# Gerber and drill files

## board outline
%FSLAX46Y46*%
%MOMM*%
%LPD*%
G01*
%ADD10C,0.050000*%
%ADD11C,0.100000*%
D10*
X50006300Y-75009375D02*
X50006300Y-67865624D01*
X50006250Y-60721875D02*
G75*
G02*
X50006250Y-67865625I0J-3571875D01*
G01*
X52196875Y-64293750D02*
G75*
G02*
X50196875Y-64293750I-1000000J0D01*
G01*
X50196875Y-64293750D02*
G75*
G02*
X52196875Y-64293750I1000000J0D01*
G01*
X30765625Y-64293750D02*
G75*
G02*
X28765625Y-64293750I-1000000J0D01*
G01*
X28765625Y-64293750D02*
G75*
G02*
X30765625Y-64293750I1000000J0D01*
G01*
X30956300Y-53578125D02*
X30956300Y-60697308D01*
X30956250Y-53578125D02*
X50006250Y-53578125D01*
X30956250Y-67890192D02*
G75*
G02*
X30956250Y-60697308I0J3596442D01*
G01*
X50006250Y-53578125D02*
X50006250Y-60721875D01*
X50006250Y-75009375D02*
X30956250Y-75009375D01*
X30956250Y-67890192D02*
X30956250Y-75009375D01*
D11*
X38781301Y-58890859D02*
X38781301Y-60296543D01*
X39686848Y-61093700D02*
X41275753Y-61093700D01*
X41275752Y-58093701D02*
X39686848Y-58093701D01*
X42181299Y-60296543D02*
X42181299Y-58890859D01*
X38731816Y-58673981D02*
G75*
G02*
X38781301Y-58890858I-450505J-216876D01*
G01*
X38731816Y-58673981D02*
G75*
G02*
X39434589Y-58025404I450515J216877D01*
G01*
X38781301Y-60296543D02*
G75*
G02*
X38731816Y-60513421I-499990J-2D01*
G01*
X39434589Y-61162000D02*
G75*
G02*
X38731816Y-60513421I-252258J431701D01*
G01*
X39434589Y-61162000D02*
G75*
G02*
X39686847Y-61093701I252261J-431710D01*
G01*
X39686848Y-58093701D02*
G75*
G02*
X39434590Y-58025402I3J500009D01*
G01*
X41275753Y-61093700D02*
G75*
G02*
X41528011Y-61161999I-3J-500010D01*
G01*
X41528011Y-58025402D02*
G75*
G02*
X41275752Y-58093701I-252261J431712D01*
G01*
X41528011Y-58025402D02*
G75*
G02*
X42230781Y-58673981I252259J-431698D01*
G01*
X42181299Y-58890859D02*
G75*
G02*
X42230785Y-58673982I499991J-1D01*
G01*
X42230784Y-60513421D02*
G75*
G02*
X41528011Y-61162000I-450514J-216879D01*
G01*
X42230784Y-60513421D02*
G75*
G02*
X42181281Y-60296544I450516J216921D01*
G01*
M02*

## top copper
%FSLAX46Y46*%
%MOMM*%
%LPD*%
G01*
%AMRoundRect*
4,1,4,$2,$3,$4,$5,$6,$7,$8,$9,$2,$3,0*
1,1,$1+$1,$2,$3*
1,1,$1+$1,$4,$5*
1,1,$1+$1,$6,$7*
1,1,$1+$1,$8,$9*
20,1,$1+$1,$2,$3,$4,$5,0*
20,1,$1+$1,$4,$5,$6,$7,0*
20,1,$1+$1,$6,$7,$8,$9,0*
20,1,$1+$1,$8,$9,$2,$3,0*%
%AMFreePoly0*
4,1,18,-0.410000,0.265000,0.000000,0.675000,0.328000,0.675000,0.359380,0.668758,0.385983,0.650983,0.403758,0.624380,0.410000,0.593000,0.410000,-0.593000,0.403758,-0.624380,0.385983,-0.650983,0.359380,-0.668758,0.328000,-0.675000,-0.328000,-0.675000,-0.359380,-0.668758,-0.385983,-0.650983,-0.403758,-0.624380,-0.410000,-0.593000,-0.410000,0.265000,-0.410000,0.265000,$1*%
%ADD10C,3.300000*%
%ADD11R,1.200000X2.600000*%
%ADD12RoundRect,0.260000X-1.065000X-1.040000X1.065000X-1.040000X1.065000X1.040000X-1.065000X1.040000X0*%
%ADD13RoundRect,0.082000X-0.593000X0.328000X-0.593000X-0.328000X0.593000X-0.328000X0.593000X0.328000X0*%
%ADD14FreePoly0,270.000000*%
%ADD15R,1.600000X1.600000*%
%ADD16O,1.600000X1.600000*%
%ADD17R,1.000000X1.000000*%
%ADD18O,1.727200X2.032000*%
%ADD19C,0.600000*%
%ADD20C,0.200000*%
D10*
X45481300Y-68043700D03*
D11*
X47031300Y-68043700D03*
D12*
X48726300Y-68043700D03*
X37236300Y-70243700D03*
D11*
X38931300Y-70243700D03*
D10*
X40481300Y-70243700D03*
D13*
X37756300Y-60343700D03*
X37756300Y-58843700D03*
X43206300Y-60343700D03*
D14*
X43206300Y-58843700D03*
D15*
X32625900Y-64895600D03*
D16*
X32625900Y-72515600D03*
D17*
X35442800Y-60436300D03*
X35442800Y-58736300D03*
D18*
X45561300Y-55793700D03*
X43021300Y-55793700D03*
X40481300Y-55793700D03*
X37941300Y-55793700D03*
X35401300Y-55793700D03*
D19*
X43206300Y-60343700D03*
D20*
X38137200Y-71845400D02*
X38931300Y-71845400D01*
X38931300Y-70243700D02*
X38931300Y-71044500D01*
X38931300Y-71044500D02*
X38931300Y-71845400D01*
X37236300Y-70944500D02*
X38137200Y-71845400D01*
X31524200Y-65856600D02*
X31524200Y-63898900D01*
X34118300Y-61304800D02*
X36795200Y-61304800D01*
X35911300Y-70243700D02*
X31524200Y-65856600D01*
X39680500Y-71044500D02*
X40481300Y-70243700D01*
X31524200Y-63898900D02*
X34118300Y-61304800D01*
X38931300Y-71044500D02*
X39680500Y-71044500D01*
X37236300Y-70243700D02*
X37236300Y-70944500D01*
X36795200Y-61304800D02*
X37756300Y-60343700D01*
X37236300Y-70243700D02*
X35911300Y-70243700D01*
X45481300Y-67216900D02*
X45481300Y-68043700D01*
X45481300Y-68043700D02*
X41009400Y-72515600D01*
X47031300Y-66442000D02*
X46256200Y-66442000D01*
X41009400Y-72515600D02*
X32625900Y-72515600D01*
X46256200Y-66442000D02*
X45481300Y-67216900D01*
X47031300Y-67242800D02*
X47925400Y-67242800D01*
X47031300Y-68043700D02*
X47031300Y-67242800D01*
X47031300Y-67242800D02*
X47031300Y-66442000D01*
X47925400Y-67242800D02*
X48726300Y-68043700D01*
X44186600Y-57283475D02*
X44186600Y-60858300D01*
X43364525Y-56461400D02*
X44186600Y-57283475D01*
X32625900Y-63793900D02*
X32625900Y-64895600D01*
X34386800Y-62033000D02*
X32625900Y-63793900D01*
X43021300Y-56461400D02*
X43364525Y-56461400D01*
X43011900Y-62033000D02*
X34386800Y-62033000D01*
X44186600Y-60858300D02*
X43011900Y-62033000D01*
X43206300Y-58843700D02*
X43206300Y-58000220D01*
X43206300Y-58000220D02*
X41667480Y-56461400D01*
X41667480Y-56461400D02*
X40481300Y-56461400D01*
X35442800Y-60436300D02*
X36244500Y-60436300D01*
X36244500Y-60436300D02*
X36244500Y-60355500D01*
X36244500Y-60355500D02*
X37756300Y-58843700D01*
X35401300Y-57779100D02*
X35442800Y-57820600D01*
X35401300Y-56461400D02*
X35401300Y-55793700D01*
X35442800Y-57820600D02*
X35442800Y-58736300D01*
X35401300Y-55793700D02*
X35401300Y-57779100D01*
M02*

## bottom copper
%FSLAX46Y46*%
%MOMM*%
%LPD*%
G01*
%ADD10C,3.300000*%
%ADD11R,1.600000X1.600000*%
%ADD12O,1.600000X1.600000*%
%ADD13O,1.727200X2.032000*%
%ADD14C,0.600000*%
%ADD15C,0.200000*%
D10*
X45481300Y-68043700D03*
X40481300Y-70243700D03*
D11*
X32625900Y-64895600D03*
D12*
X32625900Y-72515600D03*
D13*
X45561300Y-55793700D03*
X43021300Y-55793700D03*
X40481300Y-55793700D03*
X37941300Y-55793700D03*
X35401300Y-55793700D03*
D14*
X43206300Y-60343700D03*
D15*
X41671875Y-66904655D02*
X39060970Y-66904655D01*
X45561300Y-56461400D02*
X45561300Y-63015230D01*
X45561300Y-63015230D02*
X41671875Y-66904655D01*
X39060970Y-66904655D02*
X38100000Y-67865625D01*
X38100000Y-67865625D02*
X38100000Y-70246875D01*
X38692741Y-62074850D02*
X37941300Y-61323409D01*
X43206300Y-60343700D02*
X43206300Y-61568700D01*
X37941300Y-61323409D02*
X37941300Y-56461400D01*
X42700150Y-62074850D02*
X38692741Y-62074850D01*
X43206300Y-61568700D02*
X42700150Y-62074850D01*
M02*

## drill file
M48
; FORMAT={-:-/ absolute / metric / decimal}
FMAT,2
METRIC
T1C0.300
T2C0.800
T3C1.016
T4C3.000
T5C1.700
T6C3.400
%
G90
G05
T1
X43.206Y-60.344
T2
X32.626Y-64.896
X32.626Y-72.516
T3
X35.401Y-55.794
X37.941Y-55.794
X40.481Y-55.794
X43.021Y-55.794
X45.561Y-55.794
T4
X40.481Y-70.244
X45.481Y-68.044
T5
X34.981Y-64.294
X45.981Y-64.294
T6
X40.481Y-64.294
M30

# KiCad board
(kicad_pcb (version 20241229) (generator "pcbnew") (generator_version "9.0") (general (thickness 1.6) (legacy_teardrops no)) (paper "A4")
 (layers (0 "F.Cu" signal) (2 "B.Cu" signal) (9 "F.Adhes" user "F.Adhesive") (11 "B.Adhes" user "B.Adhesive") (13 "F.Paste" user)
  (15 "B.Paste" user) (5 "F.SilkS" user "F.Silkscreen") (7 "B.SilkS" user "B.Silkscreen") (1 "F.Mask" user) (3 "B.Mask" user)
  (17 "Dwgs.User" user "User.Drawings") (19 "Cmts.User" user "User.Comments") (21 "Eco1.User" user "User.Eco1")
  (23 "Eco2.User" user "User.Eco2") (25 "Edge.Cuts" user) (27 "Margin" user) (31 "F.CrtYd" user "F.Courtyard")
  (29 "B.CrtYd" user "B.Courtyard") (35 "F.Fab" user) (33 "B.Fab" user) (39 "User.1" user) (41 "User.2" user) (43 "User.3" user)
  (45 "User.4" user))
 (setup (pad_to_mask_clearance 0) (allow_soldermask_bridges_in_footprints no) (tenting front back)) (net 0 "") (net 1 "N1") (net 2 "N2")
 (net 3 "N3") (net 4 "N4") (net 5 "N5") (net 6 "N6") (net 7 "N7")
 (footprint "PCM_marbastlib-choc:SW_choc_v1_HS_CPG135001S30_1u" (layer "F.Cu") (at 40.4813 64.2937)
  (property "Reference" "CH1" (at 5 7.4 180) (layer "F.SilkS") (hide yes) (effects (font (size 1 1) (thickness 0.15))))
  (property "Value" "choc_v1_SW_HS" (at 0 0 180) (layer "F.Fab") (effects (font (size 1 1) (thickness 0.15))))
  (pad "" np_thru_hole circle (at -5.5 0 180) (size 1.7 1.7) (drill 1.7) (layers "*.Cu" "*.Mask"))
  (pad "" np_thru_hole circle (at 0 0 180) (size 3.4 3.4) (drill 3.4) (layers "*.Cu" "*.Mask"))
  (pad "" np_thru_hole circle (at 5.5 0 180) (size 1.7 1.7) (drill 1.7) (layers "*.Cu" "*.Mask"))
  (pad "1" thru_hole circle (at 5 3.75) (size 3.3 3.3) (drill 3) (layers "*.Cu" "F.Mask") (remove_unused_layers no) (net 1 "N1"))
  (pad "1" smd rect (at 6.55 3.75) (size 1.2 2.6) (layers "F.Cu") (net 1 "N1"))
  (pad "1" smd roundrect (at 8.245 3.75) (size 2.65 2.6) (layers "F.Cu" "F.Mask" "F.Paste") (roundrect_rratio 0.1) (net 1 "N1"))
  (pad "2" smd roundrect (at -3.245 5.95) (size 2.65 2.6) (layers "F.Cu" "F.Mask" "F.Paste") (roundrect_rratio 0.1) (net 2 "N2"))
  (pad "2" smd rect (at -1.55 5.95 180) (size 1.2 2.6) (layers "F.Cu") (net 2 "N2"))
  (pad "2" thru_hole circle (at 0 5.95) (size 3.3 3.3) (drill 3) (layers "*.Cu" "F.Mask") (remove_unused_layers no) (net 2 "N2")))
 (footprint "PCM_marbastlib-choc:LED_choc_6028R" (layer "F.Cu") (at 40.4813 59.5937)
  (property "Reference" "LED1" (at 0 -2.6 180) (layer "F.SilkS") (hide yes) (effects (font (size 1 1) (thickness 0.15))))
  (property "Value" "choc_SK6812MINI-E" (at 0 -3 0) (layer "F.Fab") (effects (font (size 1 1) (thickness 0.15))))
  (fp_line (start -1.699999 -0.702841) (end -1.699999 0.702843) (stroke (width 0.1) (type solid)) (layer "Edge.Cuts"))
  (fp_line (start -0.794452 1.5) (end 0.794453 1.5) (stroke (width 0.1) (type solid)) (layer "Edge.Cuts"))
  (fp_line (start 0.794452 -1.499999) (end -0.794452 -1.499999) (stroke (width 0.1) (type solid)) (layer "Edge.Cuts"))
  (fp_line (start 1.699999 0.702843) (end 1.699999 -0.702841) (stroke (width 0.1) (type solid)) (layer "Edge.Cuts"))
  (fp_arc (start -1.749484 -0.919719) (mid -1.712527 -0.814067) (end -1.699999 -0.702842) (stroke (width 0.1) (type solid))
   (layer "Edge.Cuts"))
  (fp_arc (start -1.749484 -0.919719) (mid -1.63807 -1.504033) (end -1.046711 -1.568296) (stroke (width 0.1) (type solid))
   (layer "Edge.Cuts"))
  (fp_arc (start -1.699999 0.702843) (mid -1.712527 0.814069) (end -1.749484 0.919721) (stroke (width 0.1) (type solid)) (layer "Edge.Cuts"))
  (fp_arc (start -1.046711 1.5683) (mid -1.638071 1.504036) (end -1.749484 0.919721) (stroke (width 0.1) (type solid)) (layer "Edge.Cuts"))
  (fp_arc (start -1.046711 1.5683) (mid -0.925123 1.517378) (end -0.794453 1.500001) (stroke (width 0.1) (type solid)) (layer "Edge.Cuts"))
  (fp_arc (start -0.794452 -1.499999) (mid -0.925122 -1.517376) (end -1.04671 -1.568298) (stroke (width 0.1) (type solid))
   (layer "Edge.Cuts"))
  (fp_arc (start 0.794453 1.5) (mid 0.925123 1.517377) (end 1.046711 1.568299) (stroke (width 0.1) (type solid)) (layer "Edge.Cuts"))
  (fp_arc (start 1.046711 -1.568298) (mid 0.925123 -1.517376) (end 0.794452 -1.499999) (stroke (width 0.1) (type solid)) (layer "Edge.Cuts"))
  (fp_arc (start 1.046711 -1.568298) (mid 1.638072 -1.504034) (end 1.749484 -0.919718) (stroke (width 0.1) (type solid)) (layer "Edge.Cuts"))
  (fp_arc (start 1.699999 -0.702841) (mid 1.712527 -0.814067) (end 1.749484 -0.919719) (stroke (width 0.1) (type solid)) (layer "Edge.Cuts"))
  (fp_arc (start 1.749484 0.919721) (mid 1.638071 1.504035) (end 1.046711 1.568299) (stroke (width 0.1) (type solid)) (layer "Edge.Cuts"))
  (fp_arc (start 1.749484 0.919721) (mid 1.712527 0.814069) (end 1.699999 0.702844) (stroke (width 0.1) (type solid)) (layer "Edge.Cuts"))
  (pad "1" smd roundrect (at -2.725 0.75 270) (size 0.82 1.35) (layers "F.Cu" "F.Mask" "F.Paste") (roundrect_rratio 0.1) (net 2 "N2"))
  (pad "2" smd roundrect (at -2.725 -0.75 270) (size 0.82 1.35) (layers "F.Cu" "F.Mask" "F.Paste") (roundrect_rratio 0.1) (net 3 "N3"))
  (pad "3" smd roundrect (at 2.725 0.75 270) (size 0.82 1.35) (layers "F.Cu" "F.Mask" "F.Paste") (roundrect_rratio 0.1) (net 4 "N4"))
  (pad "4" smd roundrect (at 2.725 -0.75 270) (size 0.82 1.35) (layers "F.Cu" "F.Mask" "F.Paste") (roundrect_rratio 0.1) (chamfer_ratio 0.5)
   (chamfer top_left) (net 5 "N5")))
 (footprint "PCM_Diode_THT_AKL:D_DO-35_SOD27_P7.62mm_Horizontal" (layer "F.Cu") (at 32.6259 64.8956 -90)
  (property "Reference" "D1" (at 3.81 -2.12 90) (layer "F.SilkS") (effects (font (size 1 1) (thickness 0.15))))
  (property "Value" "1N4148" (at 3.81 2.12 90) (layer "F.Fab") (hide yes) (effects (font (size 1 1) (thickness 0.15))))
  (pad "1" thru_hole rect (at 0 0 270) (size 1.6 1.6) (drill 0.8) (layers "*.Cu" "*.Mask") (remove_unused_layers no) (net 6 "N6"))
  (pad "2" thru_hole oval (at 7.62 0 270) (size 1.6 1.6) (drill 0.8) (layers "*.Cu" "*.Mask") (remove_unused_layers no) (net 1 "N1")))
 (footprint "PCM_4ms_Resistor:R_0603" (layer "F.Cu") (at 35.4428 59.5863 90)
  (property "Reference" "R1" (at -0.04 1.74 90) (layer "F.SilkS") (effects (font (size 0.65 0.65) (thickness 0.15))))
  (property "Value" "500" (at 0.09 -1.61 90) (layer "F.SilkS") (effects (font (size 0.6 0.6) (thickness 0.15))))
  (pad "1" smd rect (at -0.85 0 90) (size 1 1) (layers "F.Cu" "F.Mask" "F.Paste") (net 3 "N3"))
  (pad "2" smd rect (at 0.85 0 90) (size 1 1) (layers "F.Cu" "F.Mask" "F.Paste") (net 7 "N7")))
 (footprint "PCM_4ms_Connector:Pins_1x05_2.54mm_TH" (layer "B.Cu") (at 40.4813 55.7937 90)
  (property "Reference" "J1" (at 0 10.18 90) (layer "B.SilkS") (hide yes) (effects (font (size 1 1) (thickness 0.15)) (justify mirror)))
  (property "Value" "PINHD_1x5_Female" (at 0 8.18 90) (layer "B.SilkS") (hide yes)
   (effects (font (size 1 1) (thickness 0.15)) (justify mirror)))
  (pad "1" thru_hole oval (at 0 5.08 90) (size 2.032 1.7272) (drill 1.016) (layers "*.Cu" "*.Mask") (remove_unused_layers no) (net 2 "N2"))
  (pad "2" thru_hole oval (at 0 2.54 90) (size 2.032 1.7272) (drill 1.016) (layers "*.Cu" "*.Mask") (remove_unused_layers no) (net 6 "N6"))
  (pad "3" thru_hole oval (at 0 0 90) (size 2.032 1.7272) (drill 1.016) (layers "*.Cu" "*.Mask") (remove_unused_layers no) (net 5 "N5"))
  (pad "4" thru_hole oval (at 0 -2.54 90) (size 2.032 1.7272) (drill 1.016) (layers "*.Cu" "*.Mask") (remove_unused_layers no) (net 4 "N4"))
  (pad "5" thru_hole oval (at 0 -5.08 90) (size 2.032 1.7272) (drill 1.016) (layers "*.Cu" "*.Mask") (remove_unused_layers no) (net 7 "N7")))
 (gr_line (start 50.0063 75.009375) (end 50.0063 67.865624) (stroke (width 0.05) (type default)) (layer "Edge.Cuts"))
 (gr_arc (start 50.00625 60.721875) (mid 53.578125 64.29375) (end 50.00625 67.865625) (stroke (width 0.05) (type default))
  (layer "Edge.Cuts"))
 (gr_circle (center 51.196875 64.29375) (end 52.196875 64.29375) (stroke (width 0.05) (type solid)) (fill no) (layer "Edge.Cuts"))
 (gr_circle (center 29.765625 64.29375) (end 30.765625 64.29375) (stroke (width 0.05) (type solid)) (fill no) (layer "Edge.Cuts"))
 (gr_line (start 30.9563 53.578125) (end 30.9563 60.697308) (stroke (width 0.05) (type default)) (layer "Edge.Cuts"))
 (gr_line (start 30.95625 53.578125) (end 50.00625 53.578125) (stroke (width 0.05) (type default)) (layer "Edge.Cuts"))
 (gr_arc (start 30.95625 67.890192) (mid 27.359808 64.29375) (end 30.95625 60.697308) (stroke (width 0.05) (type default))
  (layer "Edge.Cuts"))
 (gr_line (start 50.00625 53.578125) (end 50.00625 60.721875) (stroke (width 0.05) (type default)) (layer "Edge.Cuts"))
 (gr_line (start 50.00625 75.009375) (end 30.95625 75.009375) (stroke (width 0.05) (type default)) (layer "Edge.Cuts"))
 (gr_line (start 30.95625 67.890192) (end 30.95625 75.009375) (stroke (width 0.05) (type default)) (layer "Edge.Cuts"))
 (segment (start 38.1372 71.8454) (end 38.9313 71.8454) (width 0.2) (layer "F.Cu") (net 2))
 (segment (start 38.9313 70.2437) (end 38.9313 71.0445) (width 0.2) (layer "F.Cu") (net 2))
 (segment (start 38.9313 71.0445) (end 38.9313 71.8454) (width 0.2) (layer "F.Cu") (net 2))
 (segment (start 37.2363 70.9445) (end 38.1372 71.8454) (width 0.2) (layer "F.Cu") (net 2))
 (segment (start 31.5242 65.8566) (end 31.5242 63.8989) (width 0.2) (layer "F.Cu") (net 2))
 (segment (start 34.1183 61.3048) (end 36.7952 61.3048) (width 0.2) (layer "F.Cu") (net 2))
 (segment (start 35.9113 70.2437) (end 31.5242 65.8566) (width 0.2) (layer "F.Cu") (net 2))
 (segment (start 39.6805 71.0445) (end 40.4813 70.2437) (width 0.2) (layer "F.Cu") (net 2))
 (segment (start 31.5242 63.8989) (end 34.1183 61.3048) (width 0.2) (layer "F.Cu") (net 2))
 (segment (start 38.9313 71.0445) (end 39.6805 71.0445) (width 0.2) (layer "F.Cu") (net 2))
 (segment (start 37.2363 70.2437) (end 37.2363 70.9445) (width 0.2) (layer "F.Cu") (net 2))
 (segment (start 36.7952 61.3048) (end 37.7563 60.3437) (width 0.2) (layer "F.Cu") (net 2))
 (segment (start 37.2363 70.2437) (end 35.9113 70.2437) (width 0.2) (layer "F.Cu") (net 2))
 (segment (start 41.671875 66.904655) (end 39.06097 66.904655) (width 0.2) (layer "B.Cu") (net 2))
 (segment (start 45.5613 56.4614) (end 45.5613 63.01523) (width 0.2) (layer "B.Cu") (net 2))
 (segment (start 45.5613 63.01523) (end 41.671875 66.904655) (width 0.2) (layer "B.Cu") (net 2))
 (segment (start 39.06097 66.904655) (end 38.1 67.865625) (width 0.2) (layer "B.Cu") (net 2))
 (segment (start 38.1 67.865625) (end 38.1 70.246875) (width 0.2) (layer "B.Cu") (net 2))
 (segment (start 45.4813 67.2169) (end 45.4813 68.0437) (width 0.2) (layer "F.Cu") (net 1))
 (segment (start 45.4813 68.0437) (end 41.0094 72.5156) (width 0.2) (layer "F.Cu") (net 1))
 (segment (start 47.0313 66.442) (end 46.2562 66.442) (width 0.2) (layer "F.Cu") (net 1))
 (segment (start 41.0094 72.5156) (end 32.6259 72.5156) (width 0.2) (layer "F.Cu") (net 1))
 (segment (start 46.2562 66.442) (end 45.4813 67.2169) (width 0.2) (layer "F.Cu") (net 1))
 (segment (start 47.0313 67.2428) (end 47.9254 67.2428) (width 0.2) (layer "F.Cu") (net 1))
 (segment (start 47.0313 68.0437) (end 47.0313 67.2428) (width 0.2) (layer "F.Cu") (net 1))
 (segment (start 47.0313 67.2428) (end 47.0313 66.442) (width 0.2) (layer "F.Cu") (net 1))
 (segment (start 47.9254 67.2428) (end 48.7263 68.0437) (width 0.2) (layer "F.Cu") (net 1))
 (segment (start 44.1866 57.283475) (end 44.1866 60.8583) (width 0.2) (layer "F.Cu") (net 6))
 (segment (start 43.364525 56.4614) (end 44.1866 57.283475) (width 0.2) (layer "F.Cu") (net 6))
 (segment (start 32.6259 63.7939) (end 32.6259 64.8956) (width 0.2) (layer "F.Cu") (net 6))
 (segment (start 34.3868 62.033) (end 32.6259 63.7939) (width 0.2) (layer "F.Cu") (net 6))
 (segment (start 43.0213 56.4614) (end 43.364525 56.4614) (width 0.2) (layer "F.Cu") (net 6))
 (segment (start 43.0119 62.033) (end 34.3868 62.033) (width 0.2) (layer "F.Cu") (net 6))
 (segment (start 44.1866 60.8583) (end 43.0119 62.033) (width 0.2) (layer "F.Cu") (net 6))
 (segment (start 43.2063 58.8437) (end 43.2063 58.00022) (width 0.2) (layer "F.Cu") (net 5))
 (segment (start 43.2063 58.00022) (end 41.66748 56.4614) (width 0.2) (layer "F.Cu") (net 5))
 (segment (start 41.66748 56.4614) (end 40.4813 56.4614) (width 0.2) (layer "F.Cu") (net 5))
 (segment (start 35.4428 60.4363) (end 36.2445 60.4363) (width 0.2) (layer "F.Cu") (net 3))
 (segment (start 36.2445 60.4363) (end 36.2445 60.3555) (width 0.2) (layer "F.Cu") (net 3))
 (segment (start 36.2445 60.3555) (end 37.7563 58.8437) (width 0.2) (layer "F.Cu") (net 3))
 (via (at 43.2063 60.3437) (size 0.6) (drill 0.3) (layers "F.Cu" "B.Cu") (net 4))
 (segment (start 38.692741 62.07485) (end 37.9413 61.323409) (width 0.2) (layer "B.Cu") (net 4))
 (segment (start 43.2063 60.3437) (end 43.2063 61.5687) (width 0.2) (layer "B.Cu") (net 4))
 (segment (start 37.9413 61.323409) (end 37.9413 56.4614) (width 0.2) (layer "B.Cu") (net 4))
 (segment (start 42.70015 62.07485) (end 38.692741 62.07485) (width 0.2) (layer "B.Cu") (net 4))
 (segment (start 43.2063 61.5687) (end 42.70015 62.07485) (width 0.2) (layer "B.Cu") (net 4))
 (segment (start 35.4013 57.7791) (end 35.4428 57.8206) (width 0.2) (layer "F.Cu") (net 7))
 (segment (start 35.4013 56.4614) (end 35.4013 55.7937) (width 0.2) (layer "F.Cu") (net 7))
 (segment (start 35.4428 57.8206) (end 35.4428 58.7363) (width 0.2) (layer "F.Cu") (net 7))
 (segment (start 35.4013 55.7937) (end 35.4013 57.7791) (width 0.2) (layer "F.Cu") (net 7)))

